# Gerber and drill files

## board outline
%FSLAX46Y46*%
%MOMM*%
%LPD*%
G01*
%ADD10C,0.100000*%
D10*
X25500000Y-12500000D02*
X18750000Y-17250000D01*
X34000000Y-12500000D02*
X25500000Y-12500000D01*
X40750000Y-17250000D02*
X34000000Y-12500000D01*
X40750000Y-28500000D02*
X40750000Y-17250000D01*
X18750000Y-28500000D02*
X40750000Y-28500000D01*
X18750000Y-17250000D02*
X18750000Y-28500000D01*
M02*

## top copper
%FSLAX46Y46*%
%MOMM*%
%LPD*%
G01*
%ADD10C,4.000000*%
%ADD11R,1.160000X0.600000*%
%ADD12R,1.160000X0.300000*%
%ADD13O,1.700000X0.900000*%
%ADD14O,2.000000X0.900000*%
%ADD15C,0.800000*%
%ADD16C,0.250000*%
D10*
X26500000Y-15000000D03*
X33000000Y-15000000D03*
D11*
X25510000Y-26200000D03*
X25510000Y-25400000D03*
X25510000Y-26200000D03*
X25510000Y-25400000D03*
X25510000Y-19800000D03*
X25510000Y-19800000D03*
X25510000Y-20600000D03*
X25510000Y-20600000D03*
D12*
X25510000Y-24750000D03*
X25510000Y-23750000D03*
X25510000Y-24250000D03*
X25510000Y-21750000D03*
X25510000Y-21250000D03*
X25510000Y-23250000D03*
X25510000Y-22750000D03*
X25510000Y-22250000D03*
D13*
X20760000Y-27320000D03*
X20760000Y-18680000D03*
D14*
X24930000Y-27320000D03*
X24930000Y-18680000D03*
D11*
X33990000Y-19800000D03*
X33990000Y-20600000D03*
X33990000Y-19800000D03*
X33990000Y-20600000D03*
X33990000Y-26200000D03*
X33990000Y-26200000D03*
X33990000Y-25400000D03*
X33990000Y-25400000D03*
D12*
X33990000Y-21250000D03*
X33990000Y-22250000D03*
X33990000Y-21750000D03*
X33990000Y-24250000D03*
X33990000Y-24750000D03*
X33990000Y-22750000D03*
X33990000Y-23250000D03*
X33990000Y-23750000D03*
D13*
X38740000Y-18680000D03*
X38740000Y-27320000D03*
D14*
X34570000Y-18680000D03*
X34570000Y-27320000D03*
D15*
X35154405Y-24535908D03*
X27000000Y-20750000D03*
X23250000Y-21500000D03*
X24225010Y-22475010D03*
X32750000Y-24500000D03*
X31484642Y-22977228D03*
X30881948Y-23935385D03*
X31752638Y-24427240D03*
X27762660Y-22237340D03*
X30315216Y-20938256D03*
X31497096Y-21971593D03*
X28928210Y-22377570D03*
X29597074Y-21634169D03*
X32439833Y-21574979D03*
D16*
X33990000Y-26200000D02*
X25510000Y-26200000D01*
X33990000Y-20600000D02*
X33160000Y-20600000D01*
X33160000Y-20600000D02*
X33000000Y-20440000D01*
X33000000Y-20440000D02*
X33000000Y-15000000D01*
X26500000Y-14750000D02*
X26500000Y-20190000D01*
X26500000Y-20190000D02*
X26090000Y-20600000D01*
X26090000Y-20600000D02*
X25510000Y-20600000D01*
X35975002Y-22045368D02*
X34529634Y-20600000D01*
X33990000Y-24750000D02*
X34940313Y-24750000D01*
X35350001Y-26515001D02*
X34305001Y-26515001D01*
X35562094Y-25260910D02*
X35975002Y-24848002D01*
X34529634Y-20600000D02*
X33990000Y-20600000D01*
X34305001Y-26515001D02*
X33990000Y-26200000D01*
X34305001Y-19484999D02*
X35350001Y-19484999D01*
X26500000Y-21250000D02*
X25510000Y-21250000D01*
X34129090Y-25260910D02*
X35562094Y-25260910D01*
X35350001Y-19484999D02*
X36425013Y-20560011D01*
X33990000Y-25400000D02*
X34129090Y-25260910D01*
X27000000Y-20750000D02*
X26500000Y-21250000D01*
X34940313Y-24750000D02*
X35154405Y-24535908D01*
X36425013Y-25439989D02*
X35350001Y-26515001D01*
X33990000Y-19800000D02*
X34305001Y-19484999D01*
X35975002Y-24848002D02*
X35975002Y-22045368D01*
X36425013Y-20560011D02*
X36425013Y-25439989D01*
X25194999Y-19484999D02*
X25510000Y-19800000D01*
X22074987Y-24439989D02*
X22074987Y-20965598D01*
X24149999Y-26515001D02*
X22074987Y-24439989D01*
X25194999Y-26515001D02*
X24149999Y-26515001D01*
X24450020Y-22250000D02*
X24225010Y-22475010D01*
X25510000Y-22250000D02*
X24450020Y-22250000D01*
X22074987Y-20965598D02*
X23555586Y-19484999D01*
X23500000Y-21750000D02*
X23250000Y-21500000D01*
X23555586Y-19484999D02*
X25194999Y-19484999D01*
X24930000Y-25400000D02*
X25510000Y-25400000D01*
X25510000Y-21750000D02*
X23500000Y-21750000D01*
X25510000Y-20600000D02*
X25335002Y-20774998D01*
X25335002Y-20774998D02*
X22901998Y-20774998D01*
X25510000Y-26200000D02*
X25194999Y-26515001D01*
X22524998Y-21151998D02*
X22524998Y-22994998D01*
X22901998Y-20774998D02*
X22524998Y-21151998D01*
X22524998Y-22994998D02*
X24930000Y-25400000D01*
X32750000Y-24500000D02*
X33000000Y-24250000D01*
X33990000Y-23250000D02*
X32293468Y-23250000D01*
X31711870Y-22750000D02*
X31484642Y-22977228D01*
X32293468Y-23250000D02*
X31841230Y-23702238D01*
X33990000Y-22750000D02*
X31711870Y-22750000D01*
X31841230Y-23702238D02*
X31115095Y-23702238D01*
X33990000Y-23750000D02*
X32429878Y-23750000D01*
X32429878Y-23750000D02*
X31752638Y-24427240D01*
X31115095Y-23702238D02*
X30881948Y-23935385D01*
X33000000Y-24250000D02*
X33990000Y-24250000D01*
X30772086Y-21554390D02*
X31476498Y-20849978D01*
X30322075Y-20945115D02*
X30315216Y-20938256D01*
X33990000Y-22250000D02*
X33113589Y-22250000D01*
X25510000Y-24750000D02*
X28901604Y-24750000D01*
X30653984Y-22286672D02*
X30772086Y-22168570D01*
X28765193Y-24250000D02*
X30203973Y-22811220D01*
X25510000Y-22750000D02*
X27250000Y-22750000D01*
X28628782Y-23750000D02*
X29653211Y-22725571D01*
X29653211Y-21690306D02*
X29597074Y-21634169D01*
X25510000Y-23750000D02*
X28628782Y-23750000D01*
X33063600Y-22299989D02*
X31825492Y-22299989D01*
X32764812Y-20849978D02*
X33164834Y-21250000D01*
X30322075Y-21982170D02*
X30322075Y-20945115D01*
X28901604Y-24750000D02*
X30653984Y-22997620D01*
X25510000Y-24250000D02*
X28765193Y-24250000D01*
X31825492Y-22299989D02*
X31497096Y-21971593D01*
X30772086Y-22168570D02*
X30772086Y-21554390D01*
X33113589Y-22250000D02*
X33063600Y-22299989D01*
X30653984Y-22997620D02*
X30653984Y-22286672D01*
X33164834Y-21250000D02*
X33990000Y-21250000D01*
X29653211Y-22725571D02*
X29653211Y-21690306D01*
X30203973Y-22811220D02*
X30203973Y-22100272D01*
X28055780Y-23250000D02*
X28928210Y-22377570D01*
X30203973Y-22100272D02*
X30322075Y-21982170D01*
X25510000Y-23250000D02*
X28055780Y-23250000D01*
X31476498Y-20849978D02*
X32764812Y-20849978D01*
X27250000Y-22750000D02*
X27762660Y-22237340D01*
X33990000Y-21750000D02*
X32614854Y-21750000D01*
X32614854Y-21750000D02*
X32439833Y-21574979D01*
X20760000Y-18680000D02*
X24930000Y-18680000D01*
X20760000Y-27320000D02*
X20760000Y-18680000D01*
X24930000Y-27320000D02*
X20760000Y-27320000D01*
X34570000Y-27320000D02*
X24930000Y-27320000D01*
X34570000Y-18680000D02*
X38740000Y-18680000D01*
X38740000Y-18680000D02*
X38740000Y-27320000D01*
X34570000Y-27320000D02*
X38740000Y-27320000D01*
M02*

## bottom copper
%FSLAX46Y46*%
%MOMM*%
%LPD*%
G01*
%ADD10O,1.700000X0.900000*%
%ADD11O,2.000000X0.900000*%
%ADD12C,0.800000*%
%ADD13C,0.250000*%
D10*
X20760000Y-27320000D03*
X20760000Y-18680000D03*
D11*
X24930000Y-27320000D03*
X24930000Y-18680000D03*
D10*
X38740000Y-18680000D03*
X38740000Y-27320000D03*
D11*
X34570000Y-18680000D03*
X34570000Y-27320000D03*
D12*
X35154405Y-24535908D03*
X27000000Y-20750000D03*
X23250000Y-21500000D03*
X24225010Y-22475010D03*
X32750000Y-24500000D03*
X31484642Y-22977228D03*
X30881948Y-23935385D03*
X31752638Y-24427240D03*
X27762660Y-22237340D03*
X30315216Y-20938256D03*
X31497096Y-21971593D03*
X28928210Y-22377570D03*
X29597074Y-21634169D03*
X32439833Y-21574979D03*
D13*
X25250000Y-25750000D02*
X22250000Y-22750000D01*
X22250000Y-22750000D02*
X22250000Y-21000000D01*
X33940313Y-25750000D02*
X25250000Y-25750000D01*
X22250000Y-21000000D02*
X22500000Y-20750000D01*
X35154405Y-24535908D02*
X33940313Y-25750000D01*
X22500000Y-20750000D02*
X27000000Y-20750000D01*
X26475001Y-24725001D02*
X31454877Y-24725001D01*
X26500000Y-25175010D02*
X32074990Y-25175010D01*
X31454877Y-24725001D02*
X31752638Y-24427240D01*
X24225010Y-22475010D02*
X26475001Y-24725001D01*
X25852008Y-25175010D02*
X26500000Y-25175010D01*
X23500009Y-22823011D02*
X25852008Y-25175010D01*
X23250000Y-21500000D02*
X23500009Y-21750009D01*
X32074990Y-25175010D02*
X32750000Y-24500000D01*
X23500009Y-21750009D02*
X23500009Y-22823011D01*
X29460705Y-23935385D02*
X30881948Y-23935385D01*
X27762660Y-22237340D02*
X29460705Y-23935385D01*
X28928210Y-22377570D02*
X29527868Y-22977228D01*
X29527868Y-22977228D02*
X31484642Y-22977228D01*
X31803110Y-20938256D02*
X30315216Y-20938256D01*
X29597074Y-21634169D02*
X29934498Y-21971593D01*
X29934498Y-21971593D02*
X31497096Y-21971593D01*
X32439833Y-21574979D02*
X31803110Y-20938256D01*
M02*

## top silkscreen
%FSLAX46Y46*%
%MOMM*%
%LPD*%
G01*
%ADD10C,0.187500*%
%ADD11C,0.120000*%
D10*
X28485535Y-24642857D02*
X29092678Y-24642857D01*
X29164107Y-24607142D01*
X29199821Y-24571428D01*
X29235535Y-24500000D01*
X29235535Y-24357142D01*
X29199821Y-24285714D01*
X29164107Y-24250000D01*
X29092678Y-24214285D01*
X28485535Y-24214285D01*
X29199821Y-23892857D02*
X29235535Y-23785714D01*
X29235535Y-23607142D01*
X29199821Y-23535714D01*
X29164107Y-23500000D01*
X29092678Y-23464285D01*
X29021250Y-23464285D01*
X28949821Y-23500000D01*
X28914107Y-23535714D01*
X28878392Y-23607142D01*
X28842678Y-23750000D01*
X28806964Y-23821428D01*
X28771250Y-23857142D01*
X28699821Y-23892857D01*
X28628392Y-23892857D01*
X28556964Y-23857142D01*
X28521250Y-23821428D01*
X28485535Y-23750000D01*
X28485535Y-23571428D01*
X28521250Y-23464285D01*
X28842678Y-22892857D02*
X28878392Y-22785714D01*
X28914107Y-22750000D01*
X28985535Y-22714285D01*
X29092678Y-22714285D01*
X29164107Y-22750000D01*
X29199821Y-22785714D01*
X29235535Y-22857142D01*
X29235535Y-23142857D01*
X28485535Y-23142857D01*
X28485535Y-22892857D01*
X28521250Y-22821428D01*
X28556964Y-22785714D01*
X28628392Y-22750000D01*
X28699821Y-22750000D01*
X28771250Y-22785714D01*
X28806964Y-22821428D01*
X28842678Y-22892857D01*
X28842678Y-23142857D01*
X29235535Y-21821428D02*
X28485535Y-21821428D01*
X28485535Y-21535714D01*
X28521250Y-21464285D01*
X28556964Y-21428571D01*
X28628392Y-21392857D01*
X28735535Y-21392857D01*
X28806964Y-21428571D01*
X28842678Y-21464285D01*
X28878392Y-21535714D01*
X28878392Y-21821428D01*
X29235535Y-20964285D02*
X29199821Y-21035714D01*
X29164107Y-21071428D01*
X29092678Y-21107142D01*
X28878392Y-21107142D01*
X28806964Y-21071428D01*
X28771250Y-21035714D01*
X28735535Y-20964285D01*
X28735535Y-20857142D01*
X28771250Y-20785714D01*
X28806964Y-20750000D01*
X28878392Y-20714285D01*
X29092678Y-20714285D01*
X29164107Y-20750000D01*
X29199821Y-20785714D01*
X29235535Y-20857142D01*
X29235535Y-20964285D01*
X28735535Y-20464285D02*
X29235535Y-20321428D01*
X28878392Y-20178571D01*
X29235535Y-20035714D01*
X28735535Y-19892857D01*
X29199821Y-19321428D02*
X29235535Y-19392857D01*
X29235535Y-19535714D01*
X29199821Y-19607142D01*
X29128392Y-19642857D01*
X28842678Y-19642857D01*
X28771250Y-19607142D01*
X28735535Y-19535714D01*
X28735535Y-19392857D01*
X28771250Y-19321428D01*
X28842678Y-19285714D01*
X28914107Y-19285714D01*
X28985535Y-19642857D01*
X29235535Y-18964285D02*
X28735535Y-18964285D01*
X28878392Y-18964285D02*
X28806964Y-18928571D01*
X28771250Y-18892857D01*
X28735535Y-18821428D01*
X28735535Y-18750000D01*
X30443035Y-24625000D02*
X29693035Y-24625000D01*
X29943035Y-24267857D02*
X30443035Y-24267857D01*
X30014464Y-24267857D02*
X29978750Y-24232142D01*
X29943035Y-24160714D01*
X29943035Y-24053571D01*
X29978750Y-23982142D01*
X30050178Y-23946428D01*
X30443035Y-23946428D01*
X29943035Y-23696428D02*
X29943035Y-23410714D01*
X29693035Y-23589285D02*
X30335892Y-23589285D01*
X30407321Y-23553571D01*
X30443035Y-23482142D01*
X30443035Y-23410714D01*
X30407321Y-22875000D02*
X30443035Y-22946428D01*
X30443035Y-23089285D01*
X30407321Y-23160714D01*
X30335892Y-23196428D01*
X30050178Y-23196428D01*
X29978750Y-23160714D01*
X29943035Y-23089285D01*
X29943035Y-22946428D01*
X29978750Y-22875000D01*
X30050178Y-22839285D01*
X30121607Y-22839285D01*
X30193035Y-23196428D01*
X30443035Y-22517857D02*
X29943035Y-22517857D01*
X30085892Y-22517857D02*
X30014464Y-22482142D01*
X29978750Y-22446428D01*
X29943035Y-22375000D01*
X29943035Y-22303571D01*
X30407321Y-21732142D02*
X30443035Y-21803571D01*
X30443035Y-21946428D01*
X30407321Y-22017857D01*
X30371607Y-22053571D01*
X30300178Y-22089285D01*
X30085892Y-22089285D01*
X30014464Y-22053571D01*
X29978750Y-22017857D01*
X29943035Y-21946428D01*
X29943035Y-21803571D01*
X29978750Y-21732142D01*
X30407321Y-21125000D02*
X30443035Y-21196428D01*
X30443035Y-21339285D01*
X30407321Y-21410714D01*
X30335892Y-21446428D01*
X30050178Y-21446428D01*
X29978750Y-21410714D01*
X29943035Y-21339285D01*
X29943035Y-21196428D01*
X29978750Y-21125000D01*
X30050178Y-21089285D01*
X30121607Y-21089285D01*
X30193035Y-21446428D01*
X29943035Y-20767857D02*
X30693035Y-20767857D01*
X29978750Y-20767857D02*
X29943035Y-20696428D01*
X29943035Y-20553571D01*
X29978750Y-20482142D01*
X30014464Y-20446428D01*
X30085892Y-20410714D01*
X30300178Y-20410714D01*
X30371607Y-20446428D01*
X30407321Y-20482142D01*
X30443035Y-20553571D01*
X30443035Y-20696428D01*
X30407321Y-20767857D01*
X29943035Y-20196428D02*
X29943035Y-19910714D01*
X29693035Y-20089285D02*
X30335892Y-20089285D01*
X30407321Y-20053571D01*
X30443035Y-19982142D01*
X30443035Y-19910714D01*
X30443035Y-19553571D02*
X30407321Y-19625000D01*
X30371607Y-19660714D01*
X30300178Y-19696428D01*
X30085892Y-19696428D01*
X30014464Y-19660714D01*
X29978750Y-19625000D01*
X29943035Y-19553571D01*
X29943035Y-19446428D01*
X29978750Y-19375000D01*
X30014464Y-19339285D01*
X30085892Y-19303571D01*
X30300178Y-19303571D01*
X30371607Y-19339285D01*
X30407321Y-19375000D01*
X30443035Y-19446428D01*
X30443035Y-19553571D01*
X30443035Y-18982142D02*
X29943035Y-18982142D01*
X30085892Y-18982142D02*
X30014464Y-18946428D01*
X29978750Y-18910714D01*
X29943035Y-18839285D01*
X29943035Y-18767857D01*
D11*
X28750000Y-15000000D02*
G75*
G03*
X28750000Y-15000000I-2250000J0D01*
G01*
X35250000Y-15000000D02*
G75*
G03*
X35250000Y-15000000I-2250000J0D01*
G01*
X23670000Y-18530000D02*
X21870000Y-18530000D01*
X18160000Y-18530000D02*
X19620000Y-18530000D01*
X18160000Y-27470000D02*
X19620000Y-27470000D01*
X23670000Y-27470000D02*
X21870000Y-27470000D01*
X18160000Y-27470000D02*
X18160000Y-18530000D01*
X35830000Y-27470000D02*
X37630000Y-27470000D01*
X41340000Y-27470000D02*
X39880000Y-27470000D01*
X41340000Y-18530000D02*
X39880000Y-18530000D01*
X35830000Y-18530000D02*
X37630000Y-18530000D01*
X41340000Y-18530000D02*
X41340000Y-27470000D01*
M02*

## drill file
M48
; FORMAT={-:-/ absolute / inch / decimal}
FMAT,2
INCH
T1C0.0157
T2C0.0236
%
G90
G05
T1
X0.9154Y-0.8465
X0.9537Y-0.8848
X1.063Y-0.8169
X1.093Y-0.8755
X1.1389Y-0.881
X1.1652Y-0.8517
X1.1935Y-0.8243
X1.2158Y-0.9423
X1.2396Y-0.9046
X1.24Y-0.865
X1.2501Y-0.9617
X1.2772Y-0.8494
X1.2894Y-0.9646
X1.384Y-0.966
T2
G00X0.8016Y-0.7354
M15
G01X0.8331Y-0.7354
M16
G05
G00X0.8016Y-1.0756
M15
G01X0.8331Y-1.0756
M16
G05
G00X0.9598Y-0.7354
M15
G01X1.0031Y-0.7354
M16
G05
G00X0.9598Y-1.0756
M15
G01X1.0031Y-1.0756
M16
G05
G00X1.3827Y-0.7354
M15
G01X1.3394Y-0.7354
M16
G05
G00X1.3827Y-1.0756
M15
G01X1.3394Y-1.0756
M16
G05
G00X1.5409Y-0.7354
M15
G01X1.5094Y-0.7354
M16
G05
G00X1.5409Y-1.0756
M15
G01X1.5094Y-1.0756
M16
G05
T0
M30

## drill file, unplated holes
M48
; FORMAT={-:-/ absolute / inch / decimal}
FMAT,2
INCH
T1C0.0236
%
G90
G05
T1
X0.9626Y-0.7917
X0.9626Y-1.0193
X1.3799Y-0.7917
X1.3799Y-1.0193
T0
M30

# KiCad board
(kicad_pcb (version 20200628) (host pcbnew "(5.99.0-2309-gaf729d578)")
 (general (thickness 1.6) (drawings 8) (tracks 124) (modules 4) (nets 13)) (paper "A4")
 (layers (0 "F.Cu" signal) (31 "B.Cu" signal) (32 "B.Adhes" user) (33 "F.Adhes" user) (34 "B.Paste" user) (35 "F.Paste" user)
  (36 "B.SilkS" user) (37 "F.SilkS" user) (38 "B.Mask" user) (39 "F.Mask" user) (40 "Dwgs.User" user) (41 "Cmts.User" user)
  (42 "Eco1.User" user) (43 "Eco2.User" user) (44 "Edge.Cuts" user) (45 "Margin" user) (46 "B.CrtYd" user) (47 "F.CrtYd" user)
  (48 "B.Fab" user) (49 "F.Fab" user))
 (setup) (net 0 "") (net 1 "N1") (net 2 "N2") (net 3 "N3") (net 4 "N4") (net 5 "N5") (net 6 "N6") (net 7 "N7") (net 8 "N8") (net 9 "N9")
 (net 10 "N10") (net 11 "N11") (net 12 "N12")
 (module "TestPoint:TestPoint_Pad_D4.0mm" (layer "F.Cu") (at 26.5 15)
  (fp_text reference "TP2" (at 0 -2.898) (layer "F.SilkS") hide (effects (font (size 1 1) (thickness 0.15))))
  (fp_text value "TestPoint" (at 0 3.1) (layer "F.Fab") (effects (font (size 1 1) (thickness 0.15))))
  (fp_circle (center 0 0) (end 0 2.25) (layer "F.SilkS") (width 0.12))
  (pad "1" smd circle (at 0 0) (size 4 4) (layers "F.Cu" "F.Mask") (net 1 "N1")))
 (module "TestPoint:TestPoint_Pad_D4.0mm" (layer "F.Cu") (at 33 15)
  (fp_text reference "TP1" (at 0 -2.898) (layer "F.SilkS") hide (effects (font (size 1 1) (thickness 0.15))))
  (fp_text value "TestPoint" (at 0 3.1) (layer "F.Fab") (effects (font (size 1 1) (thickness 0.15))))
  (fp_circle (center 0 0) (end 0 2.25) (layer "F.SilkS") (width 0.12))
  (pad "1" smd circle (at 0 0) (size 4 4) (layers "F.Cu" "F.Mask") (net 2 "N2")))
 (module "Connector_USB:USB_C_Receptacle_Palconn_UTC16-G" (layer "F.Cu") (at 23 23 -90)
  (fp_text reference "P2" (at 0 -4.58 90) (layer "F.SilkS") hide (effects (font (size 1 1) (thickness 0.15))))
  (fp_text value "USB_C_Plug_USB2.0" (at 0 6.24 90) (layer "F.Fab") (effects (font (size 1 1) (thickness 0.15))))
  (fp_line (start -4.47 -0.67) (end -4.47 1.13) (layer "F.SilkS") (width 0.12))
  (fp_line (start -4.47 4.84) (end -4.47 3.38) (layer "F.SilkS") (width 0.12))
  (fp_line (start 4.47 4.84) (end 4.47 3.38) (layer "F.SilkS") (width 0.12))
  (fp_line (start 4.47 -0.67) (end 4.47 1.13) (layer "F.SilkS") (width 0.12))
  (fp_line (start 4.47 4.84) (end -4.47 4.84) (layer "F.SilkS") (width 0.12))
  (pad "A12" smd rect (at 3.2 -2.51 270) (size 0.6 1.16) (layers "F.Cu" "F.Paste" "F.Mask") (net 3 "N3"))
  (pad "A9" smd rect (at 2.4 -2.51 270) (size 0.6 1.16) (layers "F.Cu" "F.Paste" "F.Mask") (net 1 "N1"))
  (pad "B1" smd rect (at 3.2 -2.51 270) (size 0.6 1.16) (layers "F.Cu" "F.Paste" "F.Mask") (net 3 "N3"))
  (pad "B4" smd rect (at 2.4 -2.51 270) (size 0.6 1.16) (layers "F.Cu" "F.Paste" "F.Mask") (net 1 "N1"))
  (pad "B12" smd rect (at -3.2 -2.51 270) (size 0.6 1.16) (layers "F.Cu" "F.Paste" "F.Mask") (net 3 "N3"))
  (pad "A1" smd rect (at -3.2 -2.51 270) (size 0.6 1.16) (layers "F.Cu" "F.Paste" "F.Mask") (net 3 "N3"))
  (pad "B9" smd rect (at -2.4 -2.51 270) (size 0.6 1.16) (layers "F.Cu" "F.Paste" "F.Mask") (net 1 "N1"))
  (pad "A4" smd rect (at -2.4 -2.51 270) (size 0.6 1.16) (layers "F.Cu" "F.Paste" "F.Mask") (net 1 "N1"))
  (pad "" np_thru_hole circle (at -2.89 -1.45 90) (size 0.6 0.6) (drill 0.6) (layers *.Cu *.Mask))
  (pad "" np_thru_hole circle (at 2.89 -1.45 90) (size 0.6 0.6) (drill 0.6) (layers *.Cu *.Mask))
  (pad "B5" smd rect (at 1.75 -2.51 90) (size 0.3 1.16) (layers "F.Cu" "F.Paste" "F.Mask") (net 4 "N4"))
  (pad "B6" smd rect (at 0.75 -2.51 90) (size 0.3 1.16) (layers "F.Cu" "F.Paste" "F.Mask") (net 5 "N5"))
  (pad "A8" smd rect (at 1.25 -2.51 90) (size 0.3 1.16) (layers "F.Cu" "F.Paste" "F.Mask") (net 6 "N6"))
  (pad "A5" smd rect (at -1.25 -2.51 90) (size 0.3 1.16) (layers "F.Cu" "F.Paste" "F.Mask") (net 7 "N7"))
  (pad "B8" smd rect (at -1.75 -2.51 90) (size 0.3 1.16) (layers "F.Cu" "F.Paste" "F.Mask") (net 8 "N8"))
  (pad "A7" smd rect (at 0.25 -2.51 90) (size 0.3 1.16) (layers "F.Cu" "F.Paste" "F.Mask") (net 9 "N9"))
  (pad "A6" smd rect (at -0.25 -2.51 90) (size 0.3 1.16) (layers "F.Cu" "F.Paste" "F.Mask") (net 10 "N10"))
  (pad "B7" smd rect (at -0.75 -2.51 90) (size 0.3 1.16) (layers "F.Cu" "F.Paste" "F.Mask") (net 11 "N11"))
  (pad "S1" thru_hole oval (at 4.32 2.24) (size 1.7 0.9) (drill oval 1.4 0.6) (layers *.Cu *.Mask) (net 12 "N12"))
  (pad "S1" thru_hole oval (at -4.32 2.24) (size 1.7 0.9) (drill oval 1.4 0.6) (layers *.Cu *.Mask) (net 12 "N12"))
  (pad "S1" thru_hole oval (at 4.32 -1.93) (size 2 0.9) (drill oval 1.7 0.6) (layers *.Cu *.Mask) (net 12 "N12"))
  (pad "S1" thru_hole oval (at -4.32 -1.93) (size 2 0.9) (drill oval 1.7 0.6) (layers *.Cu *.Mask) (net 12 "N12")))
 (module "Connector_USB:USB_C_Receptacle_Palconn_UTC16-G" (layer "F.Cu") (at 36.5 23 90)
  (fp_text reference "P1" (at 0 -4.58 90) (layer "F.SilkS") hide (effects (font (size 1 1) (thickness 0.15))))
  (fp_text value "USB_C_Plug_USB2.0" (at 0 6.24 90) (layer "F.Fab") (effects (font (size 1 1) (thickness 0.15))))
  (fp_line (start -4.47 -0.67) (end -4.47 1.13) (layer "F.SilkS") (width 0.12))
  (fp_line (start -4.47 4.84) (end -4.47 3.38) (layer "F.SilkS") (width 0.12))
  (fp_line (start 4.47 4.84) (end 4.47 3.38) (layer "F.SilkS") (width 0.12))
  (fp_line (start 4.47 -0.67) (end 4.47 1.13) (layer "F.SilkS") (width 0.12))
  (fp_line (start 4.47 4.84) (end -4.47 4.84) (layer "F.SilkS") (width 0.12))
  (pad "A12" smd rect (at 3.2 -2.51 90) (size 0.6 1.16) (layers "F.Cu" "F.Paste" "F.Mask") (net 3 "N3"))
  (pad "A9" smd rect (at 2.4 -2.51 90) (size 0.6 1.16) (layers "F.Cu" "F.Paste" "F.Mask") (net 2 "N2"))
  (pad "B1" smd rect (at 3.2 -2.51 90) (size 0.6 1.16) (layers "F.Cu" "F.Paste" "F.Mask") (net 3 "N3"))
  (pad "B4" smd rect (at 2.4 -2.51 90) (size 0.6 1.16) (layers "F.Cu" "F.Paste" "F.Mask") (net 2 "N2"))
  (pad "B12" smd rect (at -3.2 -2.51 90) (size 0.6 1.16) (layers "F.Cu" "F.Paste" "F.Mask") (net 3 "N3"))
  (pad "A1" smd rect (at -3.2 -2.51 90) (size 0.6 1.16) (layers "F.Cu" "F.Paste" "F.Mask") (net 3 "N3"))
  (pad "B9" smd rect (at -2.4 -2.51 90) (size 0.6 1.16) (layers "F.Cu" "F.Paste" "F.Mask") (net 2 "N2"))
  (pad "A4" smd rect (at -2.4 -2.51 90) (size 0.6 1.16) (layers "F.Cu" "F.Paste" "F.Mask") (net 2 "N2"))
  (pad "" np_thru_hole circle (at -2.89 -1.45 270) (size 0.6 0.6) (drill 0.6) (layers *.Cu *.Mask))
  (pad "" np_thru_hole circle (at 2.89 -1.45 270) (size 0.6 0.6) (drill 0.6) (layers *.Cu *.Mask))
  (pad "B5" smd rect (at 1.75 -2.51 270) (size 0.3 1.16) (layers "F.Cu" "F.Paste" "F.Mask") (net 4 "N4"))
  (pad "B6" smd rect (at 0.75 -2.51 270) (size 0.3 1.16) (layers "F.Cu" "F.Paste" "F.Mask") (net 5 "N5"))
  (pad "A8" smd rect (at 1.25 -2.51 270) (size 0.3 1.16) (layers "F.Cu" "F.Paste" "F.Mask") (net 6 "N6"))
  (pad "A5" smd rect (at -1.25 -2.51 270) (size 0.3 1.16) (layers "F.Cu" "F.Paste" "F.Mask") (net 7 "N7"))
  (pad "B8" smd rect (at -1.75 -2.51 270) (size 0.3 1.16) (layers "F.Cu" "F.Paste" "F.Mask") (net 8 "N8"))
  (pad "A7" smd rect (at 0.25 -2.51 270) (size 0.3 1.16) (layers "F.Cu" "F.Paste" "F.Mask") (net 9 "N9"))
  (pad "A6" smd rect (at -0.25 -2.51 270) (size 0.3 1.16) (layers "F.Cu" "F.Paste" "F.Mask") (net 10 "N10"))
  (pad "B7" smd rect (at -0.75 -2.51 270) (size 0.3 1.16) (layers "F.Cu" "F.Paste" "F.Mask") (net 11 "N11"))
  (pad "S1" thru_hole oval (at 4.32 2.24 180) (size 1.7 0.9) (drill oval 1.4 0.6) (layers *.Cu *.Mask) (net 12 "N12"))
  (pad "S1" thru_hole oval (at -4.32 2.24 180) (size 1.7 0.9) (drill oval 1.4 0.6) (layers *.Cu *.Mask) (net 12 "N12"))
  (pad "S1" thru_hole oval (at 4.32 -1.93 180) (size 2 0.9) (drill oval 1.7 0.6) (layers *.Cu *.Mask) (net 12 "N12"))
  (pad "S1" thru_hole oval (at -4.32 -1.93 180) (size 2 0.9) (drill oval 1.7 0.6) (layers *.Cu *.Mask) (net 12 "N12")))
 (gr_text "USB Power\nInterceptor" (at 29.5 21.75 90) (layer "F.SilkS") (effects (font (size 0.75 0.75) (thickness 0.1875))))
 (gr_line (start 25.5 12.5) (end 18.75 17.25) (layer "Edge.Cuts") (width 0.1))
 (gr_line (start 34 12.5) (end 25.5 12.5) (layer "Edge.Cuts") (width 0.1))
 (gr_line (start 40.75 17.25) (end 34 12.5) (layer "Edge.Cuts") (width 0.1))
 (gr_line (start 40.75 28.5) (end 40.75 17.25) (layer "Edge.Cuts") (width 0.1))
 (gr_line (start 18.75 28.5) (end 40.75 28.5) (layer "Edge.Cuts") (width 0.1))
 (gr_line (start 18.75 17.25) (end 18.75 28.5) (layer "Edge.Cuts") (width 0.1))
 (segment (start 33.99 26.2) (end 25.51 26.2) (width 0.25) (layer "F.Cu") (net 3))
 (segment (start 33.99 20.6) (end 33.16 20.6) (width 0.25) (layer "F.Cu") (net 2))
 (segment (start 33.16 20.6) (end 33 20.44) (width 0.25) (layer "F.Cu") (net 2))
 (segment (start 33 20.44) (end 33 15) (width 0.25) (layer "F.Cu") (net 2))
 (segment (start 26.5 14.75) (end 26.5 20.19) (width 0.25) (layer "F.Cu") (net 1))
 (segment (start 26.5 20.19) (end 26.09 20.6) (width 0.25) (layer "F.Cu") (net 1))
 (segment (start 26.09 20.6) (end 25.51 20.6) (width 0.25) (layer "F.Cu") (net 1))
 (segment (start 35.975002 22.045368) (end 34.529634 20.6) (width 0.25) (layer "F.Cu") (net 2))
 (segment (start 33.99 24.75) (end 34.940313 24.75) (width 0.25) (layer "F.Cu") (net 8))
 (segment (start 35.350001 26.515001) (end 34.305001 26.515001) (width 0.25) (layer "F.Cu") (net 3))
 (segment (start 35.562094 25.26091) (end 35.975002 24.848002) (width 0.25) (layer "F.Cu") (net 2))
 (segment (start 34.529634 20.6) (end 33.99 20.6) (width 0.25) (layer "F.Cu") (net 2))
 (segment (start 34.305001 26.515001) (end 33.99 26.2) (width 0.25) (layer "F.Cu") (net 3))
 (segment (start 34.305001 19.484999) (end 35.350001 19.484999) (width 0.25) (layer "F.Cu") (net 3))
 (segment (start 26.5 21.25) (end 25.51 21.25) (width 0.25) (layer "F.Cu") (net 8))
 (via (at 35.154405 24.535908) (size 0.8) (drill 0.4) (layers "F.Cu" "B.Cu") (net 8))
 (segment (start 25.25 25.75) (end 22.25 22.75) (width 0.25) (layer "B.Cu") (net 8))
 (via (at 27 20.75) (size 0.8) (drill 0.4) (layers "F.Cu" "B.Cu") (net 8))
 (segment (start 22.25 22.75) (end 22.25 21) (width 0.25) (layer "B.Cu") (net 8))
 (segment (start 34.12909 25.26091) (end 35.562094 25.26091) (width 0.25) (layer "F.Cu") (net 2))
 (segment (start 33.940313 25.75) (end 25.25 25.75) (width 0.25) (layer "B.Cu") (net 8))
 (segment (start 35.350001 19.484999) (end 36.425013 20.560011) (width 0.25) (layer "F.Cu") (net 3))
 (segment (start 33.99 25.4) (end 34.12909 25.26091) (width 0.25) (layer "F.Cu") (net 2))
 (segment (start 27 20.75) (end 26.5 21.25) (width 0.25) (layer "F.Cu") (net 8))
 (segment (start 34.940313 24.75) (end 35.154405 24.535908) (width 0.25) (layer "F.Cu") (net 8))
 (segment (start 22.25 21) (end 22.5 20.75) (width 0.25) (layer "B.Cu") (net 8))
 (segment (start 35.154405 24.535908) (end 33.940313 25.75) (width 0.25) (layer "B.Cu") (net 8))
 (segment (start 36.425013 25.439989) (end 35.350001 26.515001) (width 0.25) (layer "F.Cu") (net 3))
 (segment (start 22.5 20.75) (end 27 20.75) (width 0.25) (layer "B.Cu") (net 8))
 (segment (start 33.99 19.8) (end 34.305001 19.484999) (width 0.25) (layer "F.Cu") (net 3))
 (segment (start 35.975002 24.848002) (end 35.975002 22.045368) (width 0.25) (layer "F.Cu") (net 2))
 (segment (start 36.425013 20.560011) (end 36.425013 25.439989) (width 0.25) (layer "F.Cu") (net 3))
 (segment (start 25.194999 19.484999) (end 25.51 19.8) (width 0.25) (layer "F.Cu") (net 3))
 (segment (start 22.074987 24.439989) (end 22.074987 20.965598) (width 0.25) (layer "F.Cu") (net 3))
 (segment (start 24.149999 26.515001) (end 22.074987 24.439989) (width 0.25) (layer "F.Cu") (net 3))
 (segment (start 25.194999 26.515001) (end 24.149999 26.515001) (width 0.25) (layer "F.Cu") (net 3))
 (segment (start 24.45002 22.25) (end 24.22501 22.47501) (width 0.25) (layer "F.Cu") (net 11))
 (segment (start 25.51 22.25) (end 24.45002 22.25) (width 0.25) (layer "F.Cu") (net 11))
 (segment (start 22.074987 20.965598) (end 23.555586 19.484999) (width 0.25) (layer "F.Cu") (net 3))
 (segment (start 26.475001 24.725001) (end 31.454877 24.725001) (width 0.25) (layer "B.Cu") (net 11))
 (segment (start 23.5 21.75) (end 23.25 21.5) (width 0.25) (layer "F.Cu") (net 7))
 (segment (start 23.555586 19.484999) (end 25.194999 19.484999) (width 0.25) (layer "F.Cu") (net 3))
 (segment (start 26.5 25.17501) (end 32.07499 25.17501) (width 0.25) (layer "B.Cu") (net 7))
 (segment (start 24.93 25.4) (end 25.51 25.4) (width 0.25) (layer "F.Cu") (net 1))
 (via (at 23.25 21.5) (size 0.8) (drill 0.4) (layers "F.Cu" "B.Cu") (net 7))
 (segment (start 31.454877 24.725001) (end 31.752638 24.42724) (width 0.25) (layer "B.Cu") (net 11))
 (segment (start 24.22501 22.47501) (end 26.475001 24.725001) (width 0.25) (layer "B.Cu") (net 11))
 (segment (start 25.852008 25.17501) (end 26.5 25.17501) (width 0.25) (layer "B.Cu") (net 7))
 (segment (start 23.500009 22.823011) (end 25.852008 25.17501) (width 0.25) (layer "B.Cu") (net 7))
 (via (at 24.22501 22.47501) (size 0.8) (drill 0.4) (layers "F.Cu" "B.Cu") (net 11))
 (segment (start 23.25 21.5) (end 23.500009 21.750009) (width 0.25) (layer "B.Cu") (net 7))
 (segment (start 25.51 21.75) (end 23.5 21.75) (width 0.25) (layer "F.Cu") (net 7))
 (segment (start 25.51 20.6) (end 25.335002 20.774998) (width 0.25) (layer "F.Cu") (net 1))
 (segment (start 25.335002 20.774998) (end 22.901998 20.774998) (width 0.25) (layer "F.Cu") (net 1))
 (segment (start 25.51 26.2) (end 25.194999 26.515001) (width 0.25) (layer "F.Cu") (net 3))
 (segment (start 22.524998 21.151998) (end 22.524998 22.994998) (width 0.25) (layer "F.Cu") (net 1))
 (segment (start 32.07499 25.17501) (end 32.75 24.5) (width 0.25) (layer "B.Cu") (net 7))
 (segment (start 23.500009 21.750009) (end 23.500009 22.823011) (width 0.25) (layer "B.Cu") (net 7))
 (segment (start 22.901998 20.774998) (end 22.524998 21.151998) (width 0.25) (layer "F.Cu") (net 1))
 (segment (start 22.524998 22.994998) (end 24.93 25.4) (width 0.25) (layer "F.Cu") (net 1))
 (via (at 32.75 24.5) (size 0.8) (drill 0.4) (layers "F.Cu" "B.Cu") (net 7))
 (segment (start 32.75 24.5) (end 33 24.25) (width 0.25) (layer "F.Cu") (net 7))
 (segment (start 29.460705 23.935385) (end 30.881948 23.935385) (width 0.25) (layer "B.Cu") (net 10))
 (via (at 31.484642 22.977228) (size 0.8) (drill 0.4) (layers "F.Cu" "B.Cu") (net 9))
 (segment (start 27.76266 22.23734) (end 29.460705 23.935385) (width 0.25) (layer "B.Cu") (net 10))
 (segment (start 33.99 23.25) (end 32.293468 23.25) (width 0.25) (layer "F.Cu") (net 10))
 (segment (start 31.71187 22.75) (end 31.484642 22.977228) (width 0.25) (layer "F.Cu") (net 9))
 (via (at 30.881948 23.935385) (size 0.8) (drill 0.4) (layers "F.Cu" "B.Cu") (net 10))
 (via (at 31.752638 24.42724) (size 0.8) (drill 0.4) (layers "F.Cu" "B.Cu") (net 11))
 (segment (start 32.293468 23.25) (end 31.84123 23.702238) (width 0.25) (layer "F.Cu") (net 10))
 (segment (start 33.99 22.75) (end 31.71187 22.75) (width 0.25) (layer "F.Cu") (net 9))
 (segment (start 31.84123 23.702238) (end 31.115095 23.702238) (width 0.25) (layer "F.Cu") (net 10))
 (segment (start 28.92821 22.37757) (end 29.527868 22.977228) (width 0.25) (layer "B.Cu") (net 9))
 (segment (start 33.99 23.75) (end 32.429878 23.75) (width 0.25) (layer "F.Cu") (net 11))
 (segment (start 32.429878 23.75) (end 31.752638 24.42724) (width 0.25) (layer "F.Cu") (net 11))
 (segment (start 31.115095 23.702238) (end 30.881948 23.935385) (width 0.25) (layer "F.Cu") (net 10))
 (segment (start 29.527868 22.977228) (end 31.484642 22.977228) (width 0.25) (layer "B.Cu") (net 9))
 (segment (start 33 24.25) (end 33.99 24.25) (width 0.25) (layer "F.Cu") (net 7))
 (segment (start 30.772086 21.55439) (end 31.476498 20.849978) (width 0.25) (layer "F.Cu") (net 4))
 (segment (start 31.80311 20.938256) (end 30.315216 20.938256) (width 0.25) (layer "B.Cu") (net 6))
 (segment (start 30.322075 20.945115) (end 30.315216 20.938256) (width 0.25) (layer "F.Cu") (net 6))
 (segment (start 33.99 22.25) (end 33.113589 22.25) (width 0.25) (layer "F.Cu") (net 5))
 (via (at 27.76266 22.23734) (size 0.8) (drill 0.4) (layers "F.Cu" "B.Cu") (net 10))
 (segment (start 29.597074 21.634169) (end 29.934498 21.971593) (width 0.25) (layer "B.Cu") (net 5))
 (segment (start 25.51 24.75) (end 28.901604 24.75) (width 0.25) (layer "F.Cu") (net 4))
 (segment (start 30.653984 22.286672) (end 30.772086 22.16857) (width 0.25) (layer "F.Cu") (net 4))
 (segment (start 28.765193 24.25) (end 30.203973 22.81122) (width 0.25) (layer "F.Cu") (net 6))
 (via (at 30.315216 20.938256) (size 0.8) (drill 0.4) (layers "F.Cu" "B.Cu") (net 6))
 (segment (start 25.51 22.75) (end 27.25 22.75) (width 0.25) (layer "F.Cu") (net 10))
 (segment (start 28.628782 23.75) (end 29.653211 22.725571) (width 0.25) (layer "F.Cu") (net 5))
 (segment (start 29.653211 21.690306) (end 29.597074 21.634169) (width 0.25) (layer "F.Cu") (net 5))
 (segment (start 25.51 23.75) (end 28.628782 23.75) (width 0.25) (layer "F.Cu") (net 5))
 (via (at 31.497096 21.971593) (size 0.8) (drill 0.4) (layers "F.Cu" "B.Cu") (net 5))
 (segment (start 33.0636 22.299989) (end 31.825492 22.299989) (width 0.25) (layer "F.Cu") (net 5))
 (via (at 28.92821 22.37757) (size 0.8) (drill 0.4) (layers "F.Cu" "B.Cu") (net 9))
 (segment (start 32.764812 20.849978) (end 33.164834 21.25) (width 0.25) (layer "F.Cu") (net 4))
 (segment (start 30.322075 21.98217) (end 30.322075 20.945115) (width 0.25) (layer "F.Cu") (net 6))
 (segment (start 28.901604 24.75) (end 30.653984 22.99762) (width 0.25) (layer "F.Cu") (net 4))
 (segment (start 25.51 24.25) (end 28.765193 24.25) (width 0.25) (layer "F.Cu") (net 6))
 (segment (start 31.825492 22.299989) (end 31.497096 21.971593) (width 0.25) (layer "F.Cu") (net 5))
 (segment (start 30.772086 22.16857) (end 30.772086 21.55439) (width 0.25) (layer "F.Cu") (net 4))
 (segment (start 33.113589 22.25) (end 33.0636 22.299989) (width 0.25) (layer "F.Cu") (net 5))
 (segment (start 30.653984 22.99762) (end 30.653984 22.286672) (width 0.25) (layer "F.Cu") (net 4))
 (via (at 29.597074 21.634169) (size 0.8) (drill 0.4) (layers "F.Cu" "B.Cu") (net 5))
 (segment (start 33.164834 21.25) (end 33.99 21.25) (width 0.25) (layer "F.Cu") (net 4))
 (segment (start 29.653211 22.725571) (end 29.653211 21.690306) (width 0.25) (layer "F.Cu") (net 5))
 (segment (start 30.203973 22.81122) (end 30.203973 22.100272) (width 0.25) (layer "F.Cu") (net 6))
 (segment (start 29.934498 21.971593) (end 31.497096 21.971593) (width 0.25) (layer "B.Cu") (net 5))
 (segment (start 28.05578 23.25) (end 28.92821 22.37757) (width 0.25) (layer "F.Cu") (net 9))
 (segment (start 30.203973 22.100272) (end 30.322075 21.98217) (width 0.25) (layer "F.Cu") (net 6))
 (segment (start 25.51 23.25) (end 28.05578 23.25) (width 0.25) (layer "F.Cu") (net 9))
 (segment (start 31.476498 20.849978) (end 32.764812 20.849978) (width 0.25) (layer "F.Cu") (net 4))
 (segment (start 27.25 22.75) (end 27.76266 22.23734) (width 0.25) (layer "F.Cu") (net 10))
 (segment (start 32.439833 21.574979) (end 31.80311 20.938256) (width 0.25) (layer "B.Cu") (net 6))
 (via (at 32.439833 21.574979) (size 0.8) (drill 0.4) (layers "F.Cu" "B.Cu") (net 6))
 (segment (start 33.99 21.75) (end 32.614854 21.75) (width 0.25) (layer "F.Cu") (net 6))
 (segment (start 32.614854 21.75) (end 32.439833 21.574979) (width 0.25) (layer "F.Cu") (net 6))
 (segment (start 20.76 18.68) (end 24.93 18.68) (width 0.25) (layer "F.Cu") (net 12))
 (segment (start 20.76 27.32) (end 20.76 18.68) (width 0.25) (layer "F.Cu") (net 12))
 (segment (start 24.93 27.32) (end 20.76 27.32) (width 0.25) (layer "F.Cu") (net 12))
 (segment (start 34.57 27.32) (end 24.93 27.32) (width 0.25) (layer "F.Cu") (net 12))
 (segment (start 34.57 18.68) (end 38.74 18.68) (width 0.25) (layer "F.Cu") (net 12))
 (segment (start 38.74 18.68) (end 38.74 27.32) (width 0.25) (layer "F.Cu") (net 12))
 (segment (start 34.57 27.32) (end 38.74 27.32) (width 0.25) (layer "F.Cu") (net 12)))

